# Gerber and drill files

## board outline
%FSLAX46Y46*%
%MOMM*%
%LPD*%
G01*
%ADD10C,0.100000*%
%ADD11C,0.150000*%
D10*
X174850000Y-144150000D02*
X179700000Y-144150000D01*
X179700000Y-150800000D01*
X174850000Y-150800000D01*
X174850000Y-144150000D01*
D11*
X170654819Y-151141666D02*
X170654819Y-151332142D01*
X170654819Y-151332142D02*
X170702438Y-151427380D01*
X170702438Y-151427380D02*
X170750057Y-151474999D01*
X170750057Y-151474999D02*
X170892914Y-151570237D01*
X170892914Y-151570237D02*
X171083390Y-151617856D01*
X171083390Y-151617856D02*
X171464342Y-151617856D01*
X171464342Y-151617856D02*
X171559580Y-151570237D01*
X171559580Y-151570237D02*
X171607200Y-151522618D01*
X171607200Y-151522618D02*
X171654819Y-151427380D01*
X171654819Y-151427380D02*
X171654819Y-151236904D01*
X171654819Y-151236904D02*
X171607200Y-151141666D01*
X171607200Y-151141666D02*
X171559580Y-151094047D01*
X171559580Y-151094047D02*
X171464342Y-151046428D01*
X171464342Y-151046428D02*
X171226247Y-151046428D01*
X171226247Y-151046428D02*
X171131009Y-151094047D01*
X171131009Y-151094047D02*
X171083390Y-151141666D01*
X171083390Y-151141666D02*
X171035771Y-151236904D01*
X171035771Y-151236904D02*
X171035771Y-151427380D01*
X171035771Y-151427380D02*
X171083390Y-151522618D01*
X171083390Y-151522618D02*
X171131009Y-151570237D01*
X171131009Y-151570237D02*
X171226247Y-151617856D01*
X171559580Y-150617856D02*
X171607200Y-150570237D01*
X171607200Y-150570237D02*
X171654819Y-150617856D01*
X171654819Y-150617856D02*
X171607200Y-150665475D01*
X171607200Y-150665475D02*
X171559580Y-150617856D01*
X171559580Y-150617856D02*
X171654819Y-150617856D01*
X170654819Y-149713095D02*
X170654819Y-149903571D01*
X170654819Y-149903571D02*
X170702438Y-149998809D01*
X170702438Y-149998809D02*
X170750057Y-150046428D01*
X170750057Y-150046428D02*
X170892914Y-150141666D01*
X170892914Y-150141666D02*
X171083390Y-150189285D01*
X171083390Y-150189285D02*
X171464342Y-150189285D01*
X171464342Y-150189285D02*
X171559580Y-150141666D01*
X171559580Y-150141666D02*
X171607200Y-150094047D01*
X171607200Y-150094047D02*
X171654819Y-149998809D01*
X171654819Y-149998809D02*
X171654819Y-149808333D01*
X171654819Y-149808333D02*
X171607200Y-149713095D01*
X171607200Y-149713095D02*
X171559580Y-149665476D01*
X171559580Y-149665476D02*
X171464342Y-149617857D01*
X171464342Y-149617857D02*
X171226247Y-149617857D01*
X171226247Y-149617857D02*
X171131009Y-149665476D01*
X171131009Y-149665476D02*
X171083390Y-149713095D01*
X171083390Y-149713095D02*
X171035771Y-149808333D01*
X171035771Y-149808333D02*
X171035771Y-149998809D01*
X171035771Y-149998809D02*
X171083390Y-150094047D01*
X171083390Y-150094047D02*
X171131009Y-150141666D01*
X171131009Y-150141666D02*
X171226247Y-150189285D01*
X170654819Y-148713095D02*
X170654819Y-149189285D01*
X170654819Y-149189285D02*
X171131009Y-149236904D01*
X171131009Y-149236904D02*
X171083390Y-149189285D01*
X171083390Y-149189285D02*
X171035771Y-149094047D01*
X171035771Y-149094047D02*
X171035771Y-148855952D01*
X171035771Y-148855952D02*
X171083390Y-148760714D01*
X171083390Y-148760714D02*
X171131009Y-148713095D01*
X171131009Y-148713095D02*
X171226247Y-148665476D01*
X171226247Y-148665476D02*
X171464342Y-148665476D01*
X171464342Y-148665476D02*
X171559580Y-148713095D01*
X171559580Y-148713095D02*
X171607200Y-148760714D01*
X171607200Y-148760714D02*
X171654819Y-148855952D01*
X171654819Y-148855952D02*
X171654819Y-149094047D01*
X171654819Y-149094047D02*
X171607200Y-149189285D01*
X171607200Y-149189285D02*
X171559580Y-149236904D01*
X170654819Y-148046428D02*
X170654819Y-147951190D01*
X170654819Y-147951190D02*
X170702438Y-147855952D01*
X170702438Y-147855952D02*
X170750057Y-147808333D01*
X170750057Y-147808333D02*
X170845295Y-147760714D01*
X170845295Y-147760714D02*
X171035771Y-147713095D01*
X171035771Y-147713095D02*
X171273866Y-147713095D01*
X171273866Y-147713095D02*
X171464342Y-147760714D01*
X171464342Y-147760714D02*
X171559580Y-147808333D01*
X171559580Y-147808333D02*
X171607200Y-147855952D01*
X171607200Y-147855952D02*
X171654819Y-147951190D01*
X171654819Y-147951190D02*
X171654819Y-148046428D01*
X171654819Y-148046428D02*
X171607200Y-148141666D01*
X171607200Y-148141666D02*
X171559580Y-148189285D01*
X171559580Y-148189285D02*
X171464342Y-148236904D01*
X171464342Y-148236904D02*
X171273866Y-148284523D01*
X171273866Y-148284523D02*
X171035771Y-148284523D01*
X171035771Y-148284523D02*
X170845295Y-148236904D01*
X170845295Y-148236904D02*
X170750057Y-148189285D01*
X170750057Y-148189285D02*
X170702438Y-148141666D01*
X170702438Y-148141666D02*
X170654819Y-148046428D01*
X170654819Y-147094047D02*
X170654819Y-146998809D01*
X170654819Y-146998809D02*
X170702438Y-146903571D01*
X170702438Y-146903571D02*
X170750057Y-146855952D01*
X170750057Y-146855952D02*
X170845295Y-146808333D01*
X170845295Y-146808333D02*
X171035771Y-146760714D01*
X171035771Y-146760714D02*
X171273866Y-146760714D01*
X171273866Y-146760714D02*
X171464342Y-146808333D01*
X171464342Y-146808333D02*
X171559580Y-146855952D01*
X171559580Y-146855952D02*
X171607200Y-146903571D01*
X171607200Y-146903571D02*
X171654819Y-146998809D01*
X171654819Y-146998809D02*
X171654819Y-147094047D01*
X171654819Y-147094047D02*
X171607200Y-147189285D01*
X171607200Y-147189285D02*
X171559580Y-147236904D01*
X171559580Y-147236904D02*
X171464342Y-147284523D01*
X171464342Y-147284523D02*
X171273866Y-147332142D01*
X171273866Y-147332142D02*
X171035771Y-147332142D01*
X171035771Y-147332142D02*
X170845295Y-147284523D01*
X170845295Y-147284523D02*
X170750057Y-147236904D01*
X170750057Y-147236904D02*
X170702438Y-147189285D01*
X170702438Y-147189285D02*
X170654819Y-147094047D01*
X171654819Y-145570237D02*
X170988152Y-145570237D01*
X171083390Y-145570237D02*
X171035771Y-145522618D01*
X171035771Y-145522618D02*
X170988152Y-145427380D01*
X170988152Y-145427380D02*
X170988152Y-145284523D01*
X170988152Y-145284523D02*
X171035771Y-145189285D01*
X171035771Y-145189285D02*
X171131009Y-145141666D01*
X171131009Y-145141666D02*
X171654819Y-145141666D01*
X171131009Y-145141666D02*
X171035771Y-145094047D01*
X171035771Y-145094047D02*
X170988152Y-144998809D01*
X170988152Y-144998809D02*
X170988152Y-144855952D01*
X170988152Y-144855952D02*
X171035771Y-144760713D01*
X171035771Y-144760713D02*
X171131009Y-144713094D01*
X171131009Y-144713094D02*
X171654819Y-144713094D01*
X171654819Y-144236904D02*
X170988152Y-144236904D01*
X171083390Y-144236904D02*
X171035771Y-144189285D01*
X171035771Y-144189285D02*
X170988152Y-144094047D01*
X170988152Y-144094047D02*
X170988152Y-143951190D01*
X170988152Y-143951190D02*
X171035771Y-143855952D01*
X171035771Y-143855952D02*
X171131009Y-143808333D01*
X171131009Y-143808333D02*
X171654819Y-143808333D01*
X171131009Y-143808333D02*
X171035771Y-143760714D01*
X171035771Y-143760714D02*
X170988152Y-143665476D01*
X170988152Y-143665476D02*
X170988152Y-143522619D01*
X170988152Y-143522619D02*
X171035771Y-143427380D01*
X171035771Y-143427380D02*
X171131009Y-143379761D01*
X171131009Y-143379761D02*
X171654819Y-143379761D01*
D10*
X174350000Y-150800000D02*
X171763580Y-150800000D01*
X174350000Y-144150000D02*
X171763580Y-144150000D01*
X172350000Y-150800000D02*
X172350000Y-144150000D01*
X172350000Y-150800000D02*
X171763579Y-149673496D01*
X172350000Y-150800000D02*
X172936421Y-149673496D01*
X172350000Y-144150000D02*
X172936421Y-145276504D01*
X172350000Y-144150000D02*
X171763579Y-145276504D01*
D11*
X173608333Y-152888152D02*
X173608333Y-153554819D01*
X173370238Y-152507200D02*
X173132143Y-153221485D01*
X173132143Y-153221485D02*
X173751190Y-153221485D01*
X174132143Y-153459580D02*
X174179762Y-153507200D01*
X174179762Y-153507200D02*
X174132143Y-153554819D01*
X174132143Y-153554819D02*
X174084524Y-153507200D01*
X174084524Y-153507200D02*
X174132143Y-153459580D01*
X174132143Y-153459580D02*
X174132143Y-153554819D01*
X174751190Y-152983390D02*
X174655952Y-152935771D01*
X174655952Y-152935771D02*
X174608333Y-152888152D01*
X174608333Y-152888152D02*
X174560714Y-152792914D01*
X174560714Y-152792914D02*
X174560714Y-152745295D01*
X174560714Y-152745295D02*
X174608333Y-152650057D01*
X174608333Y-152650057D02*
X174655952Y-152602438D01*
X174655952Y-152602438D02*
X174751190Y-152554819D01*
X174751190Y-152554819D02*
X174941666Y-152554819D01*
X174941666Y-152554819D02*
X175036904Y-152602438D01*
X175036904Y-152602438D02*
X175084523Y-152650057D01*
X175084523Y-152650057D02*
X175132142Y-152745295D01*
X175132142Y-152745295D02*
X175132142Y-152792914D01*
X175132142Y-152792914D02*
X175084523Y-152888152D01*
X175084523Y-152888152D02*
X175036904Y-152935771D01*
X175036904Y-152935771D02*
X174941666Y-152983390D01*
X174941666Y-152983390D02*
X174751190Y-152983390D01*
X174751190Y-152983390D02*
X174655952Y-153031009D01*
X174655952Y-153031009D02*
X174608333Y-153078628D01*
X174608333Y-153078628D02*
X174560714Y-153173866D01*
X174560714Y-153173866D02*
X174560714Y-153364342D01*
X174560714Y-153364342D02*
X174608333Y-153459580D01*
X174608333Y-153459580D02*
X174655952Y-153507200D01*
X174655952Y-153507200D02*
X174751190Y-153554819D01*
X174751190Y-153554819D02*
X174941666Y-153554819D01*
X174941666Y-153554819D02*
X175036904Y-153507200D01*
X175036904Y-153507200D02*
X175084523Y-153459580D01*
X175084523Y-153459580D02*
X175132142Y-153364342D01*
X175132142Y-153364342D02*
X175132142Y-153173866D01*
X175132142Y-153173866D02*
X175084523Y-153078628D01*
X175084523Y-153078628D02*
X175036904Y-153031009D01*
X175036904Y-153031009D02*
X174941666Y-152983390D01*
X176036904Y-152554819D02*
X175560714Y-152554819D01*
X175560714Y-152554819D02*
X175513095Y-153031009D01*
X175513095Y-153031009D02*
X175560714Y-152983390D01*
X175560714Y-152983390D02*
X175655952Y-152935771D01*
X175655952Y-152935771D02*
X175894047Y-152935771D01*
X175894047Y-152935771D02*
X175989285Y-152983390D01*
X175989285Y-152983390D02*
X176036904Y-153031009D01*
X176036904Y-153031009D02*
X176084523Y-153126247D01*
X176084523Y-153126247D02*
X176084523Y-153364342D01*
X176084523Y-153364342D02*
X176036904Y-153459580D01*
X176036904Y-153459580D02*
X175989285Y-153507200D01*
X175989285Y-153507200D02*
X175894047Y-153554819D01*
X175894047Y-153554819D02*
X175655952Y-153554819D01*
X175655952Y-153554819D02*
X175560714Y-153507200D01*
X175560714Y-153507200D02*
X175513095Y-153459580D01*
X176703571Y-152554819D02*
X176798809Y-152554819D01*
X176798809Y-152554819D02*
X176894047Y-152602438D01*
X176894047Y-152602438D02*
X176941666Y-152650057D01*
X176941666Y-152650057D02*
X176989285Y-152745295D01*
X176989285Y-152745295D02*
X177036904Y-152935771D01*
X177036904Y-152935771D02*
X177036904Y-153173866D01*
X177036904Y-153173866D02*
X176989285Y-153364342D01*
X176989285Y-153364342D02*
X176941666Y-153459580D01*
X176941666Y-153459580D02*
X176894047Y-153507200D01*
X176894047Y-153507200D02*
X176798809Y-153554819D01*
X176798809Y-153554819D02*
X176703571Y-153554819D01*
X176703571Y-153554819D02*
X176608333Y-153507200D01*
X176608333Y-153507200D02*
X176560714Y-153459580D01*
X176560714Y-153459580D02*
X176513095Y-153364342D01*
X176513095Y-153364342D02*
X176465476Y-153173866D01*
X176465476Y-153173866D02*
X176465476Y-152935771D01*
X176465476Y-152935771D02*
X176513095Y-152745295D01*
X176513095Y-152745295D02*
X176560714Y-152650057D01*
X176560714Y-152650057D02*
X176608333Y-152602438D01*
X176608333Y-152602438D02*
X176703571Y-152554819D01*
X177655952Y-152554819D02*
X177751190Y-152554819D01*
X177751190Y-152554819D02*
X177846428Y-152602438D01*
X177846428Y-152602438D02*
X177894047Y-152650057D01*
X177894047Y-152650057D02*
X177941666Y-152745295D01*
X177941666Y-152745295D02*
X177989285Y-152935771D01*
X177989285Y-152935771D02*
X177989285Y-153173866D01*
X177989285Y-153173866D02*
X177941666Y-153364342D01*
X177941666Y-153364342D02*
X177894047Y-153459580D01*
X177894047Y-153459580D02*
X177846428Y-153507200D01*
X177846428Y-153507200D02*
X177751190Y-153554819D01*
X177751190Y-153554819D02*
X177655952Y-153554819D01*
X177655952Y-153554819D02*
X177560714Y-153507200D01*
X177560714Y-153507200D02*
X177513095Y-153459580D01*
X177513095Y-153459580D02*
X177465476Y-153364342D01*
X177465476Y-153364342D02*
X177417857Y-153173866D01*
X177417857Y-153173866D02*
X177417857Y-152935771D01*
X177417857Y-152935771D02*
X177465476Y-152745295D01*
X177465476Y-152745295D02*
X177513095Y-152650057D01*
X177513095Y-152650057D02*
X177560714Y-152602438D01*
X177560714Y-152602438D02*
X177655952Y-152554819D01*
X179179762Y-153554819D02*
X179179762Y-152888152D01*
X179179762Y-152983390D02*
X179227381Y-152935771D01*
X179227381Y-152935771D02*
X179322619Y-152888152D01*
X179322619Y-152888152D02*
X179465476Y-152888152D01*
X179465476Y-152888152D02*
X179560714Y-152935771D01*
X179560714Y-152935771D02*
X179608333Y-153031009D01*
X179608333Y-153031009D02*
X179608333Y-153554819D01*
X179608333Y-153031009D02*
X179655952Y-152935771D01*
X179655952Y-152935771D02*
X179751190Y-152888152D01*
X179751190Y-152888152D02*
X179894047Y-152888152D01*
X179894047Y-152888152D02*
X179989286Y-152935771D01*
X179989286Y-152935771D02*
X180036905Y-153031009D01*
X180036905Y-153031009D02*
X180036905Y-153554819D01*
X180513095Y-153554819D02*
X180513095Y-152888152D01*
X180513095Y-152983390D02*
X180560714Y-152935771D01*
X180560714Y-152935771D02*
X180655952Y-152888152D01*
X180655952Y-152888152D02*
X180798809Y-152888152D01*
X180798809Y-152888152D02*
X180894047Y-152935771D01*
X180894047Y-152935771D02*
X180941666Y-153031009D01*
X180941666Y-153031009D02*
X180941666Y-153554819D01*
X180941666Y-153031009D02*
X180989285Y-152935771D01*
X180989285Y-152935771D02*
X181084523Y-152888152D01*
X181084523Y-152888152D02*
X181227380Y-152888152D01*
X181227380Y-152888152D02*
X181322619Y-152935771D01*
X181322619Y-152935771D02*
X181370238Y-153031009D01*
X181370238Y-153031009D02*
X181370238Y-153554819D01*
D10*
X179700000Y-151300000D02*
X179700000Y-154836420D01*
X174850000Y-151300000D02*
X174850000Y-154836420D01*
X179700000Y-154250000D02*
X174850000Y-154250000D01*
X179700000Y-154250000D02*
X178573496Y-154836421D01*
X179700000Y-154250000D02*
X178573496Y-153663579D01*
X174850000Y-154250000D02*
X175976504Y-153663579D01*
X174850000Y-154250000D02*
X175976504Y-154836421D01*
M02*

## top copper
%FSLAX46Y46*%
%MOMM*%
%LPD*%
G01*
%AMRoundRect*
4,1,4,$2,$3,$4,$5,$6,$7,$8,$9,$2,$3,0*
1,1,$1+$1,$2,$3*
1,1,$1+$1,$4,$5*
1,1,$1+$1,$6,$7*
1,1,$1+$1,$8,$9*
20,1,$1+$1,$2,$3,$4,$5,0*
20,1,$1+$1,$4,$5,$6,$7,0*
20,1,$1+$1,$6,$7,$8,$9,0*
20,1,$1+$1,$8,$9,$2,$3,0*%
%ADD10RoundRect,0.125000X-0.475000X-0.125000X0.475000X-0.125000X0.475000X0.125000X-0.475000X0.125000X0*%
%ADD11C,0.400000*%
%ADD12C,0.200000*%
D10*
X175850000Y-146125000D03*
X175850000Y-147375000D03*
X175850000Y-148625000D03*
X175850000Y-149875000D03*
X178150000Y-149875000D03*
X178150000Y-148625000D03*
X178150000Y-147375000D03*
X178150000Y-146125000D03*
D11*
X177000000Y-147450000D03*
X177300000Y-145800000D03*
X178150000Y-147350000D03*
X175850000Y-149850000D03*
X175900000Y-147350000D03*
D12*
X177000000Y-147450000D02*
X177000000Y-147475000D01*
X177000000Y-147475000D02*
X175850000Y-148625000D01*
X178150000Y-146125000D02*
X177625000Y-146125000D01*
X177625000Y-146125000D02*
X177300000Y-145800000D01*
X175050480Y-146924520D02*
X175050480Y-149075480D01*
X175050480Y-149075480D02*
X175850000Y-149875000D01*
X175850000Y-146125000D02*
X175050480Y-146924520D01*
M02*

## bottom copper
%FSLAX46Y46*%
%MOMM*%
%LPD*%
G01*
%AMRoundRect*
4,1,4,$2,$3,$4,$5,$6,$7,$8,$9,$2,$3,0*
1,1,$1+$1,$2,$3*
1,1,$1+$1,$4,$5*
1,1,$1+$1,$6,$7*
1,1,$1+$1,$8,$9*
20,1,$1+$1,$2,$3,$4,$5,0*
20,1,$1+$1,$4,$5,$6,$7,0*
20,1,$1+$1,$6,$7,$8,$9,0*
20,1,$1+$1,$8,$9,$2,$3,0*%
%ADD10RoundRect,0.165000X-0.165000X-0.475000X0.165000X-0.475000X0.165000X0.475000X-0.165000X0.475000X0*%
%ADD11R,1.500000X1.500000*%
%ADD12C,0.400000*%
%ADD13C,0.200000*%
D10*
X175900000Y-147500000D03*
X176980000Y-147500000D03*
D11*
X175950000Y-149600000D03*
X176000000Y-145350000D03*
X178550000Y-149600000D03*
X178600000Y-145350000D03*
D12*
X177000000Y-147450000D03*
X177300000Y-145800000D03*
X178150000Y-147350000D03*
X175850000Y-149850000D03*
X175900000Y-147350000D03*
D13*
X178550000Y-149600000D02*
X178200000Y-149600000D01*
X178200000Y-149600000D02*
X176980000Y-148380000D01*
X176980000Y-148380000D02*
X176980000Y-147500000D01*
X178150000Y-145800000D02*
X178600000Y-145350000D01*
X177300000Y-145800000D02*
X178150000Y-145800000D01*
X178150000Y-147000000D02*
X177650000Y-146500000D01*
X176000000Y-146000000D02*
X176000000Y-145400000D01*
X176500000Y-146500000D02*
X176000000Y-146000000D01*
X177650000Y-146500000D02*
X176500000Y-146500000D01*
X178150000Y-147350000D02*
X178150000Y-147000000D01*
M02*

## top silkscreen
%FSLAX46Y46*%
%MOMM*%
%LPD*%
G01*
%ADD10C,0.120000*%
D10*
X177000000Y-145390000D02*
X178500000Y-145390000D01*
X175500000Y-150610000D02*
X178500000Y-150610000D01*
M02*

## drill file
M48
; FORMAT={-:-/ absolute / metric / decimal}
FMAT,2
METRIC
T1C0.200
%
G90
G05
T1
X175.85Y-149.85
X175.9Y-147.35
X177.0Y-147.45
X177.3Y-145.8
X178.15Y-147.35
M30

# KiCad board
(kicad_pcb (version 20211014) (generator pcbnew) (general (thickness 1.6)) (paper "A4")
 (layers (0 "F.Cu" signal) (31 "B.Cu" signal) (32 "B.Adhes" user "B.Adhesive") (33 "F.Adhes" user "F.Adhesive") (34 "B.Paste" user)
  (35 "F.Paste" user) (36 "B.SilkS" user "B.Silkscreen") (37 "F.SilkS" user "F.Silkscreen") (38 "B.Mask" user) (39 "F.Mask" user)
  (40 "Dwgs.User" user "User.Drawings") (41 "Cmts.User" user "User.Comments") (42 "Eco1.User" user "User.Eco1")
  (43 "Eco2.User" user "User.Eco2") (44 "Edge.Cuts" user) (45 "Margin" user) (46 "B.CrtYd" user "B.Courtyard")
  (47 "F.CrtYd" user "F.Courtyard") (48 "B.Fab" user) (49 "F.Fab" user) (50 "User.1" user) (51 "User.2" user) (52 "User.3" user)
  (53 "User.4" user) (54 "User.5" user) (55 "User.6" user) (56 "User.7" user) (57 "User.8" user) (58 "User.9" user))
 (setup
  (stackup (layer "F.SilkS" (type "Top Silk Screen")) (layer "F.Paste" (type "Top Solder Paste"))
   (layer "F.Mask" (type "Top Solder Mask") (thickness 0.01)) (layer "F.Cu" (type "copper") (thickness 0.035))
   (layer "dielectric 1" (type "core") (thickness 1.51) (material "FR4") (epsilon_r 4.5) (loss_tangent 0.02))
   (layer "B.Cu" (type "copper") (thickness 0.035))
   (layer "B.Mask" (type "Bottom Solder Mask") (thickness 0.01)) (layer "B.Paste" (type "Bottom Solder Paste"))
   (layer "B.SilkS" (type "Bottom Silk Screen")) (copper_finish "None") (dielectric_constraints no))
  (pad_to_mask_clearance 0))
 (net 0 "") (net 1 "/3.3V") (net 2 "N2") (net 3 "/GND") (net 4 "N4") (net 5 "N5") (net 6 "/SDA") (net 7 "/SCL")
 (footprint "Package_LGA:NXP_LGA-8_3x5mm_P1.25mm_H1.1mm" (layer "F.Cu") (at 177 148)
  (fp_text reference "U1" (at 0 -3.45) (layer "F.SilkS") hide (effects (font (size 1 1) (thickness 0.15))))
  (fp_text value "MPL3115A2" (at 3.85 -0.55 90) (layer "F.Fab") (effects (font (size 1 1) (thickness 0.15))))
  (fp_line (start 0 -2.61) (end 1.5 -2.61) (layer "F.SilkS") (width 0.12))
  (fp_line (start -1.5 2.61) (end 1.5 2.61) (layer "F.SilkS") (width 0.12))
  (pad "1" smd roundrect (at -1.15 -1.875) (size 1.2 0.5) (layers "F.Cu" "F.Paste" "F.Mask") (roundrect_rratio 0.25) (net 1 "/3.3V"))
  (pad "2" smd roundrect (at -1.15 -0.625) (size 1.2 0.5) (layers "F.Cu" "F.Paste" "F.Mask") (roundrect_rratio 0.25) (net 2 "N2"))
  (pad "3" smd roundrect (at -1.15 0.625) (size 1.2 0.5) (layers "F.Cu" "F.Paste" "F.Mask") (roundrect_rratio 0.25) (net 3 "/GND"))
  (pad "4" smd roundrect (at -1.15 1.875) (size 1.2 0.5) (layers "F.Cu" "F.Paste" "F.Mask") (roundrect_rratio 0.25) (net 1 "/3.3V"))
  (pad "5" smd roundrect (at 1.15 1.875) (size 1.2 0.5) (layers "F.Cu" "F.Paste" "F.Mask") (roundrect_rratio 0.25) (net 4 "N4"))
  (pad "6" smd roundrect (at 1.15 0.625) (size 1.2 0.5) (layers "F.Cu" "F.Paste" "F.Mask") (roundrect_rratio 0.25) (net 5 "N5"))
  (pad "7" smd roundrect (at 1.15 -0.625) (size 1.2 0.5) (layers "F.Cu" "F.Paste" "F.Mask") (roundrect_rratio 0.25) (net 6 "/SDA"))
  (pad "8" smd roundrect (at 1.15 -1.875) (size 1.2 0.5) (layers "F.Cu" "F.Paste" "F.Mask") (roundrect_rratio 0.25) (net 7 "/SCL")))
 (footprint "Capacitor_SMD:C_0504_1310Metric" (layer "B.Cu") (at 176.44 147.5)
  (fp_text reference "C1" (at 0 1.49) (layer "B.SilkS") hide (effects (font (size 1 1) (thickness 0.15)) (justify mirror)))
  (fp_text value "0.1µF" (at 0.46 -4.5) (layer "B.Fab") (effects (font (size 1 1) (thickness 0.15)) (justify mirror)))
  (pad "1" smd roundrect (at -0.54 0) (size 0.66 1.28) (layers "B.Cu" "B.Paste" "B.Mask") (roundrect_rratio 0.25) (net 2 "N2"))
  (pad "2" smd roundrect (at 0.54 0) (size 0.66 1.28) (layers "B.Cu" "B.Paste" "B.Mask") (roundrect_rratio 0.25) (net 3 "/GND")))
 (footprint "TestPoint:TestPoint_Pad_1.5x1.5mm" (layer "B.Cu") (at 175.95 149.6 180)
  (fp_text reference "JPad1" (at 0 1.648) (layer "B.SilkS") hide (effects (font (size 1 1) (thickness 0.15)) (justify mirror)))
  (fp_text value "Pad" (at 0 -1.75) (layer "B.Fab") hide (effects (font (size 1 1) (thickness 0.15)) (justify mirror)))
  (pad "1" smd rect (at 0 0 180) (size 1.5 1.5) (layers "B.Cu" "B.Mask") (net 1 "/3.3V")))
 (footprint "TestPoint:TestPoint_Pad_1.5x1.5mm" (layer "B.Cu") (at 176 145.35 180)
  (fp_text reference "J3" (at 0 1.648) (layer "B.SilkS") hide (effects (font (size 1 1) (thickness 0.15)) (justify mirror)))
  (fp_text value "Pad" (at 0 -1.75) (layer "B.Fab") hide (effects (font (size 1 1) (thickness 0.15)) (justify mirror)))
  (pad "1" smd rect (at 0 0 180) (size 1.5 1.5) (layers "B.Cu" "B.Mask") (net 6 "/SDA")))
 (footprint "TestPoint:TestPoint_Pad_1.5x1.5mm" (layer "B.Cu") (at 178.55 149.6 180)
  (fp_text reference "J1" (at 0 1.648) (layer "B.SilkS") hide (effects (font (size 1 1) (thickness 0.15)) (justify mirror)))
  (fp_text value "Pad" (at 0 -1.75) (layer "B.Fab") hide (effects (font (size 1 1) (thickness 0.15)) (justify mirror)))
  (pad "1" smd rect (at 0 0 180) (size 1.5 1.5) (layers "B.Cu" "B.Mask") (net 3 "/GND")))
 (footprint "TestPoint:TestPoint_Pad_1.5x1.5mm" (layer "B.Cu") (at 178.6 145.35 180)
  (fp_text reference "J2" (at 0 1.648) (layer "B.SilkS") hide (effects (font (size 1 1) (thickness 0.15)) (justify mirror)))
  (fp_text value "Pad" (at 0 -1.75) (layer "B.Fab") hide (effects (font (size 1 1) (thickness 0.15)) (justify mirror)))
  (pad "1" smd rect (at 0 0 180) (size 1.5 1.5) (layers "B.Cu" "B.Mask") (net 7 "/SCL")))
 (gr_rect (start 179.7 150.8) (end 174.85 144.15) (layer "Edge.Cuts") (width 0.1) (fill none))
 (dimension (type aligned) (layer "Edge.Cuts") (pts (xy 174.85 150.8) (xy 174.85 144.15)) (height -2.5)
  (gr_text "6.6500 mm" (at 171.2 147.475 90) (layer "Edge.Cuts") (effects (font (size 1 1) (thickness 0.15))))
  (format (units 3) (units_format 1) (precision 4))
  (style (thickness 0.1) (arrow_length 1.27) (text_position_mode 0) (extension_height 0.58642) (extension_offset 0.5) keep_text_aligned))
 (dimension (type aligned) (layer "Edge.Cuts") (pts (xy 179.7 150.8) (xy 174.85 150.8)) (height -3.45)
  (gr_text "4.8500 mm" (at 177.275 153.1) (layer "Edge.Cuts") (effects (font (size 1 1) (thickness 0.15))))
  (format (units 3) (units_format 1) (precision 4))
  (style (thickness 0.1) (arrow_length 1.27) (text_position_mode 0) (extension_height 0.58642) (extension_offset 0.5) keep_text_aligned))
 (segment (start 177 147.45) (end 177 147.475) (width 0.2) (layer "F.Cu") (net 3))
 (segment (start 177 147.475) (end 175.85 148.625) (width 0.2) (layer "F.Cu") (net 3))
 (via (at 177 147.45) (size 0.4) (drill 0.2) (layers "F.Cu" "B.Cu") (free) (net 3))
 (segment (start 178.55 149.6) (end 178.2 149.6) (width 0.2) (layer "B.Cu") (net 3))
 (segment (start 178.2 149.6) (end 176.98 148.38) (width 0.2) (layer "B.Cu") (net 3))
 (segment (start 176.98 148.38) (end 176.98 147.5) (width 0.2) (layer "B.Cu") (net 3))
 (segment (start 178.15 146.125) (end 177.625 146.125) (width 0.2) (layer "F.Cu") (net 7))
 (segment (start 177.625 146.125) (end 177.3 145.8) (width 0.2) (layer "F.Cu") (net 7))
 (via (at 177.3 145.8) (size 0.4) (drill 0.2) (layers "F.Cu" "B.Cu") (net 7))
 (segment (start 178.15 145.8) (end 178.6 145.35) (width 0.2) (layer "B.Cu") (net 7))
 (segment (start 177.3 145.8) (end 178.15 145.8) (width 0.2) (layer "B.Cu") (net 7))
 (via (at 178.15 147.35) (size 0.4) (drill 0.2) (layers "F.Cu" "B.Cu") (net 6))
 (segment (start 178.15 147) (end 177.65 146.5) (width 0.2) (layer "B.Cu") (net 6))
 (segment (start 176 146) (end 176 145.4) (width 0.2) (layer "B.Cu") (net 6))
 (segment (start 176.5 146.5) (end 176 146) (width 0.2) (layer "B.Cu") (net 6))
 (segment (start 177.65 146.5) (end 176.5 146.5) (width 0.2) (layer "B.Cu") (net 6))
 (segment (start 178.15 147.35) (end 178.15 147) (width 0.2) (layer "B.Cu") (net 6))
 (segment (start 175.05048 146.92452) (end 175.05048 149.07548) (width 0.2) (layer "F.Cu") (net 1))
 (segment (start 175.05048 149.07548) (end 175.85 149.875) (width 0.2) (layer "F.Cu") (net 1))
 (segment (start 175.85 146.125) (end 175.05048 146.92452) (width 0.2) (layer "F.Cu") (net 1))
 (via (at 175.85 149.85) (size 0.4) (drill 0.2) (layers "F.Cu" "B.Cu") (free) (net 1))
 (via (at 175.9 147.35) (size 0.4) (drill 0.2) (layers "F.Cu" "B.Cu") (free) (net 2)))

